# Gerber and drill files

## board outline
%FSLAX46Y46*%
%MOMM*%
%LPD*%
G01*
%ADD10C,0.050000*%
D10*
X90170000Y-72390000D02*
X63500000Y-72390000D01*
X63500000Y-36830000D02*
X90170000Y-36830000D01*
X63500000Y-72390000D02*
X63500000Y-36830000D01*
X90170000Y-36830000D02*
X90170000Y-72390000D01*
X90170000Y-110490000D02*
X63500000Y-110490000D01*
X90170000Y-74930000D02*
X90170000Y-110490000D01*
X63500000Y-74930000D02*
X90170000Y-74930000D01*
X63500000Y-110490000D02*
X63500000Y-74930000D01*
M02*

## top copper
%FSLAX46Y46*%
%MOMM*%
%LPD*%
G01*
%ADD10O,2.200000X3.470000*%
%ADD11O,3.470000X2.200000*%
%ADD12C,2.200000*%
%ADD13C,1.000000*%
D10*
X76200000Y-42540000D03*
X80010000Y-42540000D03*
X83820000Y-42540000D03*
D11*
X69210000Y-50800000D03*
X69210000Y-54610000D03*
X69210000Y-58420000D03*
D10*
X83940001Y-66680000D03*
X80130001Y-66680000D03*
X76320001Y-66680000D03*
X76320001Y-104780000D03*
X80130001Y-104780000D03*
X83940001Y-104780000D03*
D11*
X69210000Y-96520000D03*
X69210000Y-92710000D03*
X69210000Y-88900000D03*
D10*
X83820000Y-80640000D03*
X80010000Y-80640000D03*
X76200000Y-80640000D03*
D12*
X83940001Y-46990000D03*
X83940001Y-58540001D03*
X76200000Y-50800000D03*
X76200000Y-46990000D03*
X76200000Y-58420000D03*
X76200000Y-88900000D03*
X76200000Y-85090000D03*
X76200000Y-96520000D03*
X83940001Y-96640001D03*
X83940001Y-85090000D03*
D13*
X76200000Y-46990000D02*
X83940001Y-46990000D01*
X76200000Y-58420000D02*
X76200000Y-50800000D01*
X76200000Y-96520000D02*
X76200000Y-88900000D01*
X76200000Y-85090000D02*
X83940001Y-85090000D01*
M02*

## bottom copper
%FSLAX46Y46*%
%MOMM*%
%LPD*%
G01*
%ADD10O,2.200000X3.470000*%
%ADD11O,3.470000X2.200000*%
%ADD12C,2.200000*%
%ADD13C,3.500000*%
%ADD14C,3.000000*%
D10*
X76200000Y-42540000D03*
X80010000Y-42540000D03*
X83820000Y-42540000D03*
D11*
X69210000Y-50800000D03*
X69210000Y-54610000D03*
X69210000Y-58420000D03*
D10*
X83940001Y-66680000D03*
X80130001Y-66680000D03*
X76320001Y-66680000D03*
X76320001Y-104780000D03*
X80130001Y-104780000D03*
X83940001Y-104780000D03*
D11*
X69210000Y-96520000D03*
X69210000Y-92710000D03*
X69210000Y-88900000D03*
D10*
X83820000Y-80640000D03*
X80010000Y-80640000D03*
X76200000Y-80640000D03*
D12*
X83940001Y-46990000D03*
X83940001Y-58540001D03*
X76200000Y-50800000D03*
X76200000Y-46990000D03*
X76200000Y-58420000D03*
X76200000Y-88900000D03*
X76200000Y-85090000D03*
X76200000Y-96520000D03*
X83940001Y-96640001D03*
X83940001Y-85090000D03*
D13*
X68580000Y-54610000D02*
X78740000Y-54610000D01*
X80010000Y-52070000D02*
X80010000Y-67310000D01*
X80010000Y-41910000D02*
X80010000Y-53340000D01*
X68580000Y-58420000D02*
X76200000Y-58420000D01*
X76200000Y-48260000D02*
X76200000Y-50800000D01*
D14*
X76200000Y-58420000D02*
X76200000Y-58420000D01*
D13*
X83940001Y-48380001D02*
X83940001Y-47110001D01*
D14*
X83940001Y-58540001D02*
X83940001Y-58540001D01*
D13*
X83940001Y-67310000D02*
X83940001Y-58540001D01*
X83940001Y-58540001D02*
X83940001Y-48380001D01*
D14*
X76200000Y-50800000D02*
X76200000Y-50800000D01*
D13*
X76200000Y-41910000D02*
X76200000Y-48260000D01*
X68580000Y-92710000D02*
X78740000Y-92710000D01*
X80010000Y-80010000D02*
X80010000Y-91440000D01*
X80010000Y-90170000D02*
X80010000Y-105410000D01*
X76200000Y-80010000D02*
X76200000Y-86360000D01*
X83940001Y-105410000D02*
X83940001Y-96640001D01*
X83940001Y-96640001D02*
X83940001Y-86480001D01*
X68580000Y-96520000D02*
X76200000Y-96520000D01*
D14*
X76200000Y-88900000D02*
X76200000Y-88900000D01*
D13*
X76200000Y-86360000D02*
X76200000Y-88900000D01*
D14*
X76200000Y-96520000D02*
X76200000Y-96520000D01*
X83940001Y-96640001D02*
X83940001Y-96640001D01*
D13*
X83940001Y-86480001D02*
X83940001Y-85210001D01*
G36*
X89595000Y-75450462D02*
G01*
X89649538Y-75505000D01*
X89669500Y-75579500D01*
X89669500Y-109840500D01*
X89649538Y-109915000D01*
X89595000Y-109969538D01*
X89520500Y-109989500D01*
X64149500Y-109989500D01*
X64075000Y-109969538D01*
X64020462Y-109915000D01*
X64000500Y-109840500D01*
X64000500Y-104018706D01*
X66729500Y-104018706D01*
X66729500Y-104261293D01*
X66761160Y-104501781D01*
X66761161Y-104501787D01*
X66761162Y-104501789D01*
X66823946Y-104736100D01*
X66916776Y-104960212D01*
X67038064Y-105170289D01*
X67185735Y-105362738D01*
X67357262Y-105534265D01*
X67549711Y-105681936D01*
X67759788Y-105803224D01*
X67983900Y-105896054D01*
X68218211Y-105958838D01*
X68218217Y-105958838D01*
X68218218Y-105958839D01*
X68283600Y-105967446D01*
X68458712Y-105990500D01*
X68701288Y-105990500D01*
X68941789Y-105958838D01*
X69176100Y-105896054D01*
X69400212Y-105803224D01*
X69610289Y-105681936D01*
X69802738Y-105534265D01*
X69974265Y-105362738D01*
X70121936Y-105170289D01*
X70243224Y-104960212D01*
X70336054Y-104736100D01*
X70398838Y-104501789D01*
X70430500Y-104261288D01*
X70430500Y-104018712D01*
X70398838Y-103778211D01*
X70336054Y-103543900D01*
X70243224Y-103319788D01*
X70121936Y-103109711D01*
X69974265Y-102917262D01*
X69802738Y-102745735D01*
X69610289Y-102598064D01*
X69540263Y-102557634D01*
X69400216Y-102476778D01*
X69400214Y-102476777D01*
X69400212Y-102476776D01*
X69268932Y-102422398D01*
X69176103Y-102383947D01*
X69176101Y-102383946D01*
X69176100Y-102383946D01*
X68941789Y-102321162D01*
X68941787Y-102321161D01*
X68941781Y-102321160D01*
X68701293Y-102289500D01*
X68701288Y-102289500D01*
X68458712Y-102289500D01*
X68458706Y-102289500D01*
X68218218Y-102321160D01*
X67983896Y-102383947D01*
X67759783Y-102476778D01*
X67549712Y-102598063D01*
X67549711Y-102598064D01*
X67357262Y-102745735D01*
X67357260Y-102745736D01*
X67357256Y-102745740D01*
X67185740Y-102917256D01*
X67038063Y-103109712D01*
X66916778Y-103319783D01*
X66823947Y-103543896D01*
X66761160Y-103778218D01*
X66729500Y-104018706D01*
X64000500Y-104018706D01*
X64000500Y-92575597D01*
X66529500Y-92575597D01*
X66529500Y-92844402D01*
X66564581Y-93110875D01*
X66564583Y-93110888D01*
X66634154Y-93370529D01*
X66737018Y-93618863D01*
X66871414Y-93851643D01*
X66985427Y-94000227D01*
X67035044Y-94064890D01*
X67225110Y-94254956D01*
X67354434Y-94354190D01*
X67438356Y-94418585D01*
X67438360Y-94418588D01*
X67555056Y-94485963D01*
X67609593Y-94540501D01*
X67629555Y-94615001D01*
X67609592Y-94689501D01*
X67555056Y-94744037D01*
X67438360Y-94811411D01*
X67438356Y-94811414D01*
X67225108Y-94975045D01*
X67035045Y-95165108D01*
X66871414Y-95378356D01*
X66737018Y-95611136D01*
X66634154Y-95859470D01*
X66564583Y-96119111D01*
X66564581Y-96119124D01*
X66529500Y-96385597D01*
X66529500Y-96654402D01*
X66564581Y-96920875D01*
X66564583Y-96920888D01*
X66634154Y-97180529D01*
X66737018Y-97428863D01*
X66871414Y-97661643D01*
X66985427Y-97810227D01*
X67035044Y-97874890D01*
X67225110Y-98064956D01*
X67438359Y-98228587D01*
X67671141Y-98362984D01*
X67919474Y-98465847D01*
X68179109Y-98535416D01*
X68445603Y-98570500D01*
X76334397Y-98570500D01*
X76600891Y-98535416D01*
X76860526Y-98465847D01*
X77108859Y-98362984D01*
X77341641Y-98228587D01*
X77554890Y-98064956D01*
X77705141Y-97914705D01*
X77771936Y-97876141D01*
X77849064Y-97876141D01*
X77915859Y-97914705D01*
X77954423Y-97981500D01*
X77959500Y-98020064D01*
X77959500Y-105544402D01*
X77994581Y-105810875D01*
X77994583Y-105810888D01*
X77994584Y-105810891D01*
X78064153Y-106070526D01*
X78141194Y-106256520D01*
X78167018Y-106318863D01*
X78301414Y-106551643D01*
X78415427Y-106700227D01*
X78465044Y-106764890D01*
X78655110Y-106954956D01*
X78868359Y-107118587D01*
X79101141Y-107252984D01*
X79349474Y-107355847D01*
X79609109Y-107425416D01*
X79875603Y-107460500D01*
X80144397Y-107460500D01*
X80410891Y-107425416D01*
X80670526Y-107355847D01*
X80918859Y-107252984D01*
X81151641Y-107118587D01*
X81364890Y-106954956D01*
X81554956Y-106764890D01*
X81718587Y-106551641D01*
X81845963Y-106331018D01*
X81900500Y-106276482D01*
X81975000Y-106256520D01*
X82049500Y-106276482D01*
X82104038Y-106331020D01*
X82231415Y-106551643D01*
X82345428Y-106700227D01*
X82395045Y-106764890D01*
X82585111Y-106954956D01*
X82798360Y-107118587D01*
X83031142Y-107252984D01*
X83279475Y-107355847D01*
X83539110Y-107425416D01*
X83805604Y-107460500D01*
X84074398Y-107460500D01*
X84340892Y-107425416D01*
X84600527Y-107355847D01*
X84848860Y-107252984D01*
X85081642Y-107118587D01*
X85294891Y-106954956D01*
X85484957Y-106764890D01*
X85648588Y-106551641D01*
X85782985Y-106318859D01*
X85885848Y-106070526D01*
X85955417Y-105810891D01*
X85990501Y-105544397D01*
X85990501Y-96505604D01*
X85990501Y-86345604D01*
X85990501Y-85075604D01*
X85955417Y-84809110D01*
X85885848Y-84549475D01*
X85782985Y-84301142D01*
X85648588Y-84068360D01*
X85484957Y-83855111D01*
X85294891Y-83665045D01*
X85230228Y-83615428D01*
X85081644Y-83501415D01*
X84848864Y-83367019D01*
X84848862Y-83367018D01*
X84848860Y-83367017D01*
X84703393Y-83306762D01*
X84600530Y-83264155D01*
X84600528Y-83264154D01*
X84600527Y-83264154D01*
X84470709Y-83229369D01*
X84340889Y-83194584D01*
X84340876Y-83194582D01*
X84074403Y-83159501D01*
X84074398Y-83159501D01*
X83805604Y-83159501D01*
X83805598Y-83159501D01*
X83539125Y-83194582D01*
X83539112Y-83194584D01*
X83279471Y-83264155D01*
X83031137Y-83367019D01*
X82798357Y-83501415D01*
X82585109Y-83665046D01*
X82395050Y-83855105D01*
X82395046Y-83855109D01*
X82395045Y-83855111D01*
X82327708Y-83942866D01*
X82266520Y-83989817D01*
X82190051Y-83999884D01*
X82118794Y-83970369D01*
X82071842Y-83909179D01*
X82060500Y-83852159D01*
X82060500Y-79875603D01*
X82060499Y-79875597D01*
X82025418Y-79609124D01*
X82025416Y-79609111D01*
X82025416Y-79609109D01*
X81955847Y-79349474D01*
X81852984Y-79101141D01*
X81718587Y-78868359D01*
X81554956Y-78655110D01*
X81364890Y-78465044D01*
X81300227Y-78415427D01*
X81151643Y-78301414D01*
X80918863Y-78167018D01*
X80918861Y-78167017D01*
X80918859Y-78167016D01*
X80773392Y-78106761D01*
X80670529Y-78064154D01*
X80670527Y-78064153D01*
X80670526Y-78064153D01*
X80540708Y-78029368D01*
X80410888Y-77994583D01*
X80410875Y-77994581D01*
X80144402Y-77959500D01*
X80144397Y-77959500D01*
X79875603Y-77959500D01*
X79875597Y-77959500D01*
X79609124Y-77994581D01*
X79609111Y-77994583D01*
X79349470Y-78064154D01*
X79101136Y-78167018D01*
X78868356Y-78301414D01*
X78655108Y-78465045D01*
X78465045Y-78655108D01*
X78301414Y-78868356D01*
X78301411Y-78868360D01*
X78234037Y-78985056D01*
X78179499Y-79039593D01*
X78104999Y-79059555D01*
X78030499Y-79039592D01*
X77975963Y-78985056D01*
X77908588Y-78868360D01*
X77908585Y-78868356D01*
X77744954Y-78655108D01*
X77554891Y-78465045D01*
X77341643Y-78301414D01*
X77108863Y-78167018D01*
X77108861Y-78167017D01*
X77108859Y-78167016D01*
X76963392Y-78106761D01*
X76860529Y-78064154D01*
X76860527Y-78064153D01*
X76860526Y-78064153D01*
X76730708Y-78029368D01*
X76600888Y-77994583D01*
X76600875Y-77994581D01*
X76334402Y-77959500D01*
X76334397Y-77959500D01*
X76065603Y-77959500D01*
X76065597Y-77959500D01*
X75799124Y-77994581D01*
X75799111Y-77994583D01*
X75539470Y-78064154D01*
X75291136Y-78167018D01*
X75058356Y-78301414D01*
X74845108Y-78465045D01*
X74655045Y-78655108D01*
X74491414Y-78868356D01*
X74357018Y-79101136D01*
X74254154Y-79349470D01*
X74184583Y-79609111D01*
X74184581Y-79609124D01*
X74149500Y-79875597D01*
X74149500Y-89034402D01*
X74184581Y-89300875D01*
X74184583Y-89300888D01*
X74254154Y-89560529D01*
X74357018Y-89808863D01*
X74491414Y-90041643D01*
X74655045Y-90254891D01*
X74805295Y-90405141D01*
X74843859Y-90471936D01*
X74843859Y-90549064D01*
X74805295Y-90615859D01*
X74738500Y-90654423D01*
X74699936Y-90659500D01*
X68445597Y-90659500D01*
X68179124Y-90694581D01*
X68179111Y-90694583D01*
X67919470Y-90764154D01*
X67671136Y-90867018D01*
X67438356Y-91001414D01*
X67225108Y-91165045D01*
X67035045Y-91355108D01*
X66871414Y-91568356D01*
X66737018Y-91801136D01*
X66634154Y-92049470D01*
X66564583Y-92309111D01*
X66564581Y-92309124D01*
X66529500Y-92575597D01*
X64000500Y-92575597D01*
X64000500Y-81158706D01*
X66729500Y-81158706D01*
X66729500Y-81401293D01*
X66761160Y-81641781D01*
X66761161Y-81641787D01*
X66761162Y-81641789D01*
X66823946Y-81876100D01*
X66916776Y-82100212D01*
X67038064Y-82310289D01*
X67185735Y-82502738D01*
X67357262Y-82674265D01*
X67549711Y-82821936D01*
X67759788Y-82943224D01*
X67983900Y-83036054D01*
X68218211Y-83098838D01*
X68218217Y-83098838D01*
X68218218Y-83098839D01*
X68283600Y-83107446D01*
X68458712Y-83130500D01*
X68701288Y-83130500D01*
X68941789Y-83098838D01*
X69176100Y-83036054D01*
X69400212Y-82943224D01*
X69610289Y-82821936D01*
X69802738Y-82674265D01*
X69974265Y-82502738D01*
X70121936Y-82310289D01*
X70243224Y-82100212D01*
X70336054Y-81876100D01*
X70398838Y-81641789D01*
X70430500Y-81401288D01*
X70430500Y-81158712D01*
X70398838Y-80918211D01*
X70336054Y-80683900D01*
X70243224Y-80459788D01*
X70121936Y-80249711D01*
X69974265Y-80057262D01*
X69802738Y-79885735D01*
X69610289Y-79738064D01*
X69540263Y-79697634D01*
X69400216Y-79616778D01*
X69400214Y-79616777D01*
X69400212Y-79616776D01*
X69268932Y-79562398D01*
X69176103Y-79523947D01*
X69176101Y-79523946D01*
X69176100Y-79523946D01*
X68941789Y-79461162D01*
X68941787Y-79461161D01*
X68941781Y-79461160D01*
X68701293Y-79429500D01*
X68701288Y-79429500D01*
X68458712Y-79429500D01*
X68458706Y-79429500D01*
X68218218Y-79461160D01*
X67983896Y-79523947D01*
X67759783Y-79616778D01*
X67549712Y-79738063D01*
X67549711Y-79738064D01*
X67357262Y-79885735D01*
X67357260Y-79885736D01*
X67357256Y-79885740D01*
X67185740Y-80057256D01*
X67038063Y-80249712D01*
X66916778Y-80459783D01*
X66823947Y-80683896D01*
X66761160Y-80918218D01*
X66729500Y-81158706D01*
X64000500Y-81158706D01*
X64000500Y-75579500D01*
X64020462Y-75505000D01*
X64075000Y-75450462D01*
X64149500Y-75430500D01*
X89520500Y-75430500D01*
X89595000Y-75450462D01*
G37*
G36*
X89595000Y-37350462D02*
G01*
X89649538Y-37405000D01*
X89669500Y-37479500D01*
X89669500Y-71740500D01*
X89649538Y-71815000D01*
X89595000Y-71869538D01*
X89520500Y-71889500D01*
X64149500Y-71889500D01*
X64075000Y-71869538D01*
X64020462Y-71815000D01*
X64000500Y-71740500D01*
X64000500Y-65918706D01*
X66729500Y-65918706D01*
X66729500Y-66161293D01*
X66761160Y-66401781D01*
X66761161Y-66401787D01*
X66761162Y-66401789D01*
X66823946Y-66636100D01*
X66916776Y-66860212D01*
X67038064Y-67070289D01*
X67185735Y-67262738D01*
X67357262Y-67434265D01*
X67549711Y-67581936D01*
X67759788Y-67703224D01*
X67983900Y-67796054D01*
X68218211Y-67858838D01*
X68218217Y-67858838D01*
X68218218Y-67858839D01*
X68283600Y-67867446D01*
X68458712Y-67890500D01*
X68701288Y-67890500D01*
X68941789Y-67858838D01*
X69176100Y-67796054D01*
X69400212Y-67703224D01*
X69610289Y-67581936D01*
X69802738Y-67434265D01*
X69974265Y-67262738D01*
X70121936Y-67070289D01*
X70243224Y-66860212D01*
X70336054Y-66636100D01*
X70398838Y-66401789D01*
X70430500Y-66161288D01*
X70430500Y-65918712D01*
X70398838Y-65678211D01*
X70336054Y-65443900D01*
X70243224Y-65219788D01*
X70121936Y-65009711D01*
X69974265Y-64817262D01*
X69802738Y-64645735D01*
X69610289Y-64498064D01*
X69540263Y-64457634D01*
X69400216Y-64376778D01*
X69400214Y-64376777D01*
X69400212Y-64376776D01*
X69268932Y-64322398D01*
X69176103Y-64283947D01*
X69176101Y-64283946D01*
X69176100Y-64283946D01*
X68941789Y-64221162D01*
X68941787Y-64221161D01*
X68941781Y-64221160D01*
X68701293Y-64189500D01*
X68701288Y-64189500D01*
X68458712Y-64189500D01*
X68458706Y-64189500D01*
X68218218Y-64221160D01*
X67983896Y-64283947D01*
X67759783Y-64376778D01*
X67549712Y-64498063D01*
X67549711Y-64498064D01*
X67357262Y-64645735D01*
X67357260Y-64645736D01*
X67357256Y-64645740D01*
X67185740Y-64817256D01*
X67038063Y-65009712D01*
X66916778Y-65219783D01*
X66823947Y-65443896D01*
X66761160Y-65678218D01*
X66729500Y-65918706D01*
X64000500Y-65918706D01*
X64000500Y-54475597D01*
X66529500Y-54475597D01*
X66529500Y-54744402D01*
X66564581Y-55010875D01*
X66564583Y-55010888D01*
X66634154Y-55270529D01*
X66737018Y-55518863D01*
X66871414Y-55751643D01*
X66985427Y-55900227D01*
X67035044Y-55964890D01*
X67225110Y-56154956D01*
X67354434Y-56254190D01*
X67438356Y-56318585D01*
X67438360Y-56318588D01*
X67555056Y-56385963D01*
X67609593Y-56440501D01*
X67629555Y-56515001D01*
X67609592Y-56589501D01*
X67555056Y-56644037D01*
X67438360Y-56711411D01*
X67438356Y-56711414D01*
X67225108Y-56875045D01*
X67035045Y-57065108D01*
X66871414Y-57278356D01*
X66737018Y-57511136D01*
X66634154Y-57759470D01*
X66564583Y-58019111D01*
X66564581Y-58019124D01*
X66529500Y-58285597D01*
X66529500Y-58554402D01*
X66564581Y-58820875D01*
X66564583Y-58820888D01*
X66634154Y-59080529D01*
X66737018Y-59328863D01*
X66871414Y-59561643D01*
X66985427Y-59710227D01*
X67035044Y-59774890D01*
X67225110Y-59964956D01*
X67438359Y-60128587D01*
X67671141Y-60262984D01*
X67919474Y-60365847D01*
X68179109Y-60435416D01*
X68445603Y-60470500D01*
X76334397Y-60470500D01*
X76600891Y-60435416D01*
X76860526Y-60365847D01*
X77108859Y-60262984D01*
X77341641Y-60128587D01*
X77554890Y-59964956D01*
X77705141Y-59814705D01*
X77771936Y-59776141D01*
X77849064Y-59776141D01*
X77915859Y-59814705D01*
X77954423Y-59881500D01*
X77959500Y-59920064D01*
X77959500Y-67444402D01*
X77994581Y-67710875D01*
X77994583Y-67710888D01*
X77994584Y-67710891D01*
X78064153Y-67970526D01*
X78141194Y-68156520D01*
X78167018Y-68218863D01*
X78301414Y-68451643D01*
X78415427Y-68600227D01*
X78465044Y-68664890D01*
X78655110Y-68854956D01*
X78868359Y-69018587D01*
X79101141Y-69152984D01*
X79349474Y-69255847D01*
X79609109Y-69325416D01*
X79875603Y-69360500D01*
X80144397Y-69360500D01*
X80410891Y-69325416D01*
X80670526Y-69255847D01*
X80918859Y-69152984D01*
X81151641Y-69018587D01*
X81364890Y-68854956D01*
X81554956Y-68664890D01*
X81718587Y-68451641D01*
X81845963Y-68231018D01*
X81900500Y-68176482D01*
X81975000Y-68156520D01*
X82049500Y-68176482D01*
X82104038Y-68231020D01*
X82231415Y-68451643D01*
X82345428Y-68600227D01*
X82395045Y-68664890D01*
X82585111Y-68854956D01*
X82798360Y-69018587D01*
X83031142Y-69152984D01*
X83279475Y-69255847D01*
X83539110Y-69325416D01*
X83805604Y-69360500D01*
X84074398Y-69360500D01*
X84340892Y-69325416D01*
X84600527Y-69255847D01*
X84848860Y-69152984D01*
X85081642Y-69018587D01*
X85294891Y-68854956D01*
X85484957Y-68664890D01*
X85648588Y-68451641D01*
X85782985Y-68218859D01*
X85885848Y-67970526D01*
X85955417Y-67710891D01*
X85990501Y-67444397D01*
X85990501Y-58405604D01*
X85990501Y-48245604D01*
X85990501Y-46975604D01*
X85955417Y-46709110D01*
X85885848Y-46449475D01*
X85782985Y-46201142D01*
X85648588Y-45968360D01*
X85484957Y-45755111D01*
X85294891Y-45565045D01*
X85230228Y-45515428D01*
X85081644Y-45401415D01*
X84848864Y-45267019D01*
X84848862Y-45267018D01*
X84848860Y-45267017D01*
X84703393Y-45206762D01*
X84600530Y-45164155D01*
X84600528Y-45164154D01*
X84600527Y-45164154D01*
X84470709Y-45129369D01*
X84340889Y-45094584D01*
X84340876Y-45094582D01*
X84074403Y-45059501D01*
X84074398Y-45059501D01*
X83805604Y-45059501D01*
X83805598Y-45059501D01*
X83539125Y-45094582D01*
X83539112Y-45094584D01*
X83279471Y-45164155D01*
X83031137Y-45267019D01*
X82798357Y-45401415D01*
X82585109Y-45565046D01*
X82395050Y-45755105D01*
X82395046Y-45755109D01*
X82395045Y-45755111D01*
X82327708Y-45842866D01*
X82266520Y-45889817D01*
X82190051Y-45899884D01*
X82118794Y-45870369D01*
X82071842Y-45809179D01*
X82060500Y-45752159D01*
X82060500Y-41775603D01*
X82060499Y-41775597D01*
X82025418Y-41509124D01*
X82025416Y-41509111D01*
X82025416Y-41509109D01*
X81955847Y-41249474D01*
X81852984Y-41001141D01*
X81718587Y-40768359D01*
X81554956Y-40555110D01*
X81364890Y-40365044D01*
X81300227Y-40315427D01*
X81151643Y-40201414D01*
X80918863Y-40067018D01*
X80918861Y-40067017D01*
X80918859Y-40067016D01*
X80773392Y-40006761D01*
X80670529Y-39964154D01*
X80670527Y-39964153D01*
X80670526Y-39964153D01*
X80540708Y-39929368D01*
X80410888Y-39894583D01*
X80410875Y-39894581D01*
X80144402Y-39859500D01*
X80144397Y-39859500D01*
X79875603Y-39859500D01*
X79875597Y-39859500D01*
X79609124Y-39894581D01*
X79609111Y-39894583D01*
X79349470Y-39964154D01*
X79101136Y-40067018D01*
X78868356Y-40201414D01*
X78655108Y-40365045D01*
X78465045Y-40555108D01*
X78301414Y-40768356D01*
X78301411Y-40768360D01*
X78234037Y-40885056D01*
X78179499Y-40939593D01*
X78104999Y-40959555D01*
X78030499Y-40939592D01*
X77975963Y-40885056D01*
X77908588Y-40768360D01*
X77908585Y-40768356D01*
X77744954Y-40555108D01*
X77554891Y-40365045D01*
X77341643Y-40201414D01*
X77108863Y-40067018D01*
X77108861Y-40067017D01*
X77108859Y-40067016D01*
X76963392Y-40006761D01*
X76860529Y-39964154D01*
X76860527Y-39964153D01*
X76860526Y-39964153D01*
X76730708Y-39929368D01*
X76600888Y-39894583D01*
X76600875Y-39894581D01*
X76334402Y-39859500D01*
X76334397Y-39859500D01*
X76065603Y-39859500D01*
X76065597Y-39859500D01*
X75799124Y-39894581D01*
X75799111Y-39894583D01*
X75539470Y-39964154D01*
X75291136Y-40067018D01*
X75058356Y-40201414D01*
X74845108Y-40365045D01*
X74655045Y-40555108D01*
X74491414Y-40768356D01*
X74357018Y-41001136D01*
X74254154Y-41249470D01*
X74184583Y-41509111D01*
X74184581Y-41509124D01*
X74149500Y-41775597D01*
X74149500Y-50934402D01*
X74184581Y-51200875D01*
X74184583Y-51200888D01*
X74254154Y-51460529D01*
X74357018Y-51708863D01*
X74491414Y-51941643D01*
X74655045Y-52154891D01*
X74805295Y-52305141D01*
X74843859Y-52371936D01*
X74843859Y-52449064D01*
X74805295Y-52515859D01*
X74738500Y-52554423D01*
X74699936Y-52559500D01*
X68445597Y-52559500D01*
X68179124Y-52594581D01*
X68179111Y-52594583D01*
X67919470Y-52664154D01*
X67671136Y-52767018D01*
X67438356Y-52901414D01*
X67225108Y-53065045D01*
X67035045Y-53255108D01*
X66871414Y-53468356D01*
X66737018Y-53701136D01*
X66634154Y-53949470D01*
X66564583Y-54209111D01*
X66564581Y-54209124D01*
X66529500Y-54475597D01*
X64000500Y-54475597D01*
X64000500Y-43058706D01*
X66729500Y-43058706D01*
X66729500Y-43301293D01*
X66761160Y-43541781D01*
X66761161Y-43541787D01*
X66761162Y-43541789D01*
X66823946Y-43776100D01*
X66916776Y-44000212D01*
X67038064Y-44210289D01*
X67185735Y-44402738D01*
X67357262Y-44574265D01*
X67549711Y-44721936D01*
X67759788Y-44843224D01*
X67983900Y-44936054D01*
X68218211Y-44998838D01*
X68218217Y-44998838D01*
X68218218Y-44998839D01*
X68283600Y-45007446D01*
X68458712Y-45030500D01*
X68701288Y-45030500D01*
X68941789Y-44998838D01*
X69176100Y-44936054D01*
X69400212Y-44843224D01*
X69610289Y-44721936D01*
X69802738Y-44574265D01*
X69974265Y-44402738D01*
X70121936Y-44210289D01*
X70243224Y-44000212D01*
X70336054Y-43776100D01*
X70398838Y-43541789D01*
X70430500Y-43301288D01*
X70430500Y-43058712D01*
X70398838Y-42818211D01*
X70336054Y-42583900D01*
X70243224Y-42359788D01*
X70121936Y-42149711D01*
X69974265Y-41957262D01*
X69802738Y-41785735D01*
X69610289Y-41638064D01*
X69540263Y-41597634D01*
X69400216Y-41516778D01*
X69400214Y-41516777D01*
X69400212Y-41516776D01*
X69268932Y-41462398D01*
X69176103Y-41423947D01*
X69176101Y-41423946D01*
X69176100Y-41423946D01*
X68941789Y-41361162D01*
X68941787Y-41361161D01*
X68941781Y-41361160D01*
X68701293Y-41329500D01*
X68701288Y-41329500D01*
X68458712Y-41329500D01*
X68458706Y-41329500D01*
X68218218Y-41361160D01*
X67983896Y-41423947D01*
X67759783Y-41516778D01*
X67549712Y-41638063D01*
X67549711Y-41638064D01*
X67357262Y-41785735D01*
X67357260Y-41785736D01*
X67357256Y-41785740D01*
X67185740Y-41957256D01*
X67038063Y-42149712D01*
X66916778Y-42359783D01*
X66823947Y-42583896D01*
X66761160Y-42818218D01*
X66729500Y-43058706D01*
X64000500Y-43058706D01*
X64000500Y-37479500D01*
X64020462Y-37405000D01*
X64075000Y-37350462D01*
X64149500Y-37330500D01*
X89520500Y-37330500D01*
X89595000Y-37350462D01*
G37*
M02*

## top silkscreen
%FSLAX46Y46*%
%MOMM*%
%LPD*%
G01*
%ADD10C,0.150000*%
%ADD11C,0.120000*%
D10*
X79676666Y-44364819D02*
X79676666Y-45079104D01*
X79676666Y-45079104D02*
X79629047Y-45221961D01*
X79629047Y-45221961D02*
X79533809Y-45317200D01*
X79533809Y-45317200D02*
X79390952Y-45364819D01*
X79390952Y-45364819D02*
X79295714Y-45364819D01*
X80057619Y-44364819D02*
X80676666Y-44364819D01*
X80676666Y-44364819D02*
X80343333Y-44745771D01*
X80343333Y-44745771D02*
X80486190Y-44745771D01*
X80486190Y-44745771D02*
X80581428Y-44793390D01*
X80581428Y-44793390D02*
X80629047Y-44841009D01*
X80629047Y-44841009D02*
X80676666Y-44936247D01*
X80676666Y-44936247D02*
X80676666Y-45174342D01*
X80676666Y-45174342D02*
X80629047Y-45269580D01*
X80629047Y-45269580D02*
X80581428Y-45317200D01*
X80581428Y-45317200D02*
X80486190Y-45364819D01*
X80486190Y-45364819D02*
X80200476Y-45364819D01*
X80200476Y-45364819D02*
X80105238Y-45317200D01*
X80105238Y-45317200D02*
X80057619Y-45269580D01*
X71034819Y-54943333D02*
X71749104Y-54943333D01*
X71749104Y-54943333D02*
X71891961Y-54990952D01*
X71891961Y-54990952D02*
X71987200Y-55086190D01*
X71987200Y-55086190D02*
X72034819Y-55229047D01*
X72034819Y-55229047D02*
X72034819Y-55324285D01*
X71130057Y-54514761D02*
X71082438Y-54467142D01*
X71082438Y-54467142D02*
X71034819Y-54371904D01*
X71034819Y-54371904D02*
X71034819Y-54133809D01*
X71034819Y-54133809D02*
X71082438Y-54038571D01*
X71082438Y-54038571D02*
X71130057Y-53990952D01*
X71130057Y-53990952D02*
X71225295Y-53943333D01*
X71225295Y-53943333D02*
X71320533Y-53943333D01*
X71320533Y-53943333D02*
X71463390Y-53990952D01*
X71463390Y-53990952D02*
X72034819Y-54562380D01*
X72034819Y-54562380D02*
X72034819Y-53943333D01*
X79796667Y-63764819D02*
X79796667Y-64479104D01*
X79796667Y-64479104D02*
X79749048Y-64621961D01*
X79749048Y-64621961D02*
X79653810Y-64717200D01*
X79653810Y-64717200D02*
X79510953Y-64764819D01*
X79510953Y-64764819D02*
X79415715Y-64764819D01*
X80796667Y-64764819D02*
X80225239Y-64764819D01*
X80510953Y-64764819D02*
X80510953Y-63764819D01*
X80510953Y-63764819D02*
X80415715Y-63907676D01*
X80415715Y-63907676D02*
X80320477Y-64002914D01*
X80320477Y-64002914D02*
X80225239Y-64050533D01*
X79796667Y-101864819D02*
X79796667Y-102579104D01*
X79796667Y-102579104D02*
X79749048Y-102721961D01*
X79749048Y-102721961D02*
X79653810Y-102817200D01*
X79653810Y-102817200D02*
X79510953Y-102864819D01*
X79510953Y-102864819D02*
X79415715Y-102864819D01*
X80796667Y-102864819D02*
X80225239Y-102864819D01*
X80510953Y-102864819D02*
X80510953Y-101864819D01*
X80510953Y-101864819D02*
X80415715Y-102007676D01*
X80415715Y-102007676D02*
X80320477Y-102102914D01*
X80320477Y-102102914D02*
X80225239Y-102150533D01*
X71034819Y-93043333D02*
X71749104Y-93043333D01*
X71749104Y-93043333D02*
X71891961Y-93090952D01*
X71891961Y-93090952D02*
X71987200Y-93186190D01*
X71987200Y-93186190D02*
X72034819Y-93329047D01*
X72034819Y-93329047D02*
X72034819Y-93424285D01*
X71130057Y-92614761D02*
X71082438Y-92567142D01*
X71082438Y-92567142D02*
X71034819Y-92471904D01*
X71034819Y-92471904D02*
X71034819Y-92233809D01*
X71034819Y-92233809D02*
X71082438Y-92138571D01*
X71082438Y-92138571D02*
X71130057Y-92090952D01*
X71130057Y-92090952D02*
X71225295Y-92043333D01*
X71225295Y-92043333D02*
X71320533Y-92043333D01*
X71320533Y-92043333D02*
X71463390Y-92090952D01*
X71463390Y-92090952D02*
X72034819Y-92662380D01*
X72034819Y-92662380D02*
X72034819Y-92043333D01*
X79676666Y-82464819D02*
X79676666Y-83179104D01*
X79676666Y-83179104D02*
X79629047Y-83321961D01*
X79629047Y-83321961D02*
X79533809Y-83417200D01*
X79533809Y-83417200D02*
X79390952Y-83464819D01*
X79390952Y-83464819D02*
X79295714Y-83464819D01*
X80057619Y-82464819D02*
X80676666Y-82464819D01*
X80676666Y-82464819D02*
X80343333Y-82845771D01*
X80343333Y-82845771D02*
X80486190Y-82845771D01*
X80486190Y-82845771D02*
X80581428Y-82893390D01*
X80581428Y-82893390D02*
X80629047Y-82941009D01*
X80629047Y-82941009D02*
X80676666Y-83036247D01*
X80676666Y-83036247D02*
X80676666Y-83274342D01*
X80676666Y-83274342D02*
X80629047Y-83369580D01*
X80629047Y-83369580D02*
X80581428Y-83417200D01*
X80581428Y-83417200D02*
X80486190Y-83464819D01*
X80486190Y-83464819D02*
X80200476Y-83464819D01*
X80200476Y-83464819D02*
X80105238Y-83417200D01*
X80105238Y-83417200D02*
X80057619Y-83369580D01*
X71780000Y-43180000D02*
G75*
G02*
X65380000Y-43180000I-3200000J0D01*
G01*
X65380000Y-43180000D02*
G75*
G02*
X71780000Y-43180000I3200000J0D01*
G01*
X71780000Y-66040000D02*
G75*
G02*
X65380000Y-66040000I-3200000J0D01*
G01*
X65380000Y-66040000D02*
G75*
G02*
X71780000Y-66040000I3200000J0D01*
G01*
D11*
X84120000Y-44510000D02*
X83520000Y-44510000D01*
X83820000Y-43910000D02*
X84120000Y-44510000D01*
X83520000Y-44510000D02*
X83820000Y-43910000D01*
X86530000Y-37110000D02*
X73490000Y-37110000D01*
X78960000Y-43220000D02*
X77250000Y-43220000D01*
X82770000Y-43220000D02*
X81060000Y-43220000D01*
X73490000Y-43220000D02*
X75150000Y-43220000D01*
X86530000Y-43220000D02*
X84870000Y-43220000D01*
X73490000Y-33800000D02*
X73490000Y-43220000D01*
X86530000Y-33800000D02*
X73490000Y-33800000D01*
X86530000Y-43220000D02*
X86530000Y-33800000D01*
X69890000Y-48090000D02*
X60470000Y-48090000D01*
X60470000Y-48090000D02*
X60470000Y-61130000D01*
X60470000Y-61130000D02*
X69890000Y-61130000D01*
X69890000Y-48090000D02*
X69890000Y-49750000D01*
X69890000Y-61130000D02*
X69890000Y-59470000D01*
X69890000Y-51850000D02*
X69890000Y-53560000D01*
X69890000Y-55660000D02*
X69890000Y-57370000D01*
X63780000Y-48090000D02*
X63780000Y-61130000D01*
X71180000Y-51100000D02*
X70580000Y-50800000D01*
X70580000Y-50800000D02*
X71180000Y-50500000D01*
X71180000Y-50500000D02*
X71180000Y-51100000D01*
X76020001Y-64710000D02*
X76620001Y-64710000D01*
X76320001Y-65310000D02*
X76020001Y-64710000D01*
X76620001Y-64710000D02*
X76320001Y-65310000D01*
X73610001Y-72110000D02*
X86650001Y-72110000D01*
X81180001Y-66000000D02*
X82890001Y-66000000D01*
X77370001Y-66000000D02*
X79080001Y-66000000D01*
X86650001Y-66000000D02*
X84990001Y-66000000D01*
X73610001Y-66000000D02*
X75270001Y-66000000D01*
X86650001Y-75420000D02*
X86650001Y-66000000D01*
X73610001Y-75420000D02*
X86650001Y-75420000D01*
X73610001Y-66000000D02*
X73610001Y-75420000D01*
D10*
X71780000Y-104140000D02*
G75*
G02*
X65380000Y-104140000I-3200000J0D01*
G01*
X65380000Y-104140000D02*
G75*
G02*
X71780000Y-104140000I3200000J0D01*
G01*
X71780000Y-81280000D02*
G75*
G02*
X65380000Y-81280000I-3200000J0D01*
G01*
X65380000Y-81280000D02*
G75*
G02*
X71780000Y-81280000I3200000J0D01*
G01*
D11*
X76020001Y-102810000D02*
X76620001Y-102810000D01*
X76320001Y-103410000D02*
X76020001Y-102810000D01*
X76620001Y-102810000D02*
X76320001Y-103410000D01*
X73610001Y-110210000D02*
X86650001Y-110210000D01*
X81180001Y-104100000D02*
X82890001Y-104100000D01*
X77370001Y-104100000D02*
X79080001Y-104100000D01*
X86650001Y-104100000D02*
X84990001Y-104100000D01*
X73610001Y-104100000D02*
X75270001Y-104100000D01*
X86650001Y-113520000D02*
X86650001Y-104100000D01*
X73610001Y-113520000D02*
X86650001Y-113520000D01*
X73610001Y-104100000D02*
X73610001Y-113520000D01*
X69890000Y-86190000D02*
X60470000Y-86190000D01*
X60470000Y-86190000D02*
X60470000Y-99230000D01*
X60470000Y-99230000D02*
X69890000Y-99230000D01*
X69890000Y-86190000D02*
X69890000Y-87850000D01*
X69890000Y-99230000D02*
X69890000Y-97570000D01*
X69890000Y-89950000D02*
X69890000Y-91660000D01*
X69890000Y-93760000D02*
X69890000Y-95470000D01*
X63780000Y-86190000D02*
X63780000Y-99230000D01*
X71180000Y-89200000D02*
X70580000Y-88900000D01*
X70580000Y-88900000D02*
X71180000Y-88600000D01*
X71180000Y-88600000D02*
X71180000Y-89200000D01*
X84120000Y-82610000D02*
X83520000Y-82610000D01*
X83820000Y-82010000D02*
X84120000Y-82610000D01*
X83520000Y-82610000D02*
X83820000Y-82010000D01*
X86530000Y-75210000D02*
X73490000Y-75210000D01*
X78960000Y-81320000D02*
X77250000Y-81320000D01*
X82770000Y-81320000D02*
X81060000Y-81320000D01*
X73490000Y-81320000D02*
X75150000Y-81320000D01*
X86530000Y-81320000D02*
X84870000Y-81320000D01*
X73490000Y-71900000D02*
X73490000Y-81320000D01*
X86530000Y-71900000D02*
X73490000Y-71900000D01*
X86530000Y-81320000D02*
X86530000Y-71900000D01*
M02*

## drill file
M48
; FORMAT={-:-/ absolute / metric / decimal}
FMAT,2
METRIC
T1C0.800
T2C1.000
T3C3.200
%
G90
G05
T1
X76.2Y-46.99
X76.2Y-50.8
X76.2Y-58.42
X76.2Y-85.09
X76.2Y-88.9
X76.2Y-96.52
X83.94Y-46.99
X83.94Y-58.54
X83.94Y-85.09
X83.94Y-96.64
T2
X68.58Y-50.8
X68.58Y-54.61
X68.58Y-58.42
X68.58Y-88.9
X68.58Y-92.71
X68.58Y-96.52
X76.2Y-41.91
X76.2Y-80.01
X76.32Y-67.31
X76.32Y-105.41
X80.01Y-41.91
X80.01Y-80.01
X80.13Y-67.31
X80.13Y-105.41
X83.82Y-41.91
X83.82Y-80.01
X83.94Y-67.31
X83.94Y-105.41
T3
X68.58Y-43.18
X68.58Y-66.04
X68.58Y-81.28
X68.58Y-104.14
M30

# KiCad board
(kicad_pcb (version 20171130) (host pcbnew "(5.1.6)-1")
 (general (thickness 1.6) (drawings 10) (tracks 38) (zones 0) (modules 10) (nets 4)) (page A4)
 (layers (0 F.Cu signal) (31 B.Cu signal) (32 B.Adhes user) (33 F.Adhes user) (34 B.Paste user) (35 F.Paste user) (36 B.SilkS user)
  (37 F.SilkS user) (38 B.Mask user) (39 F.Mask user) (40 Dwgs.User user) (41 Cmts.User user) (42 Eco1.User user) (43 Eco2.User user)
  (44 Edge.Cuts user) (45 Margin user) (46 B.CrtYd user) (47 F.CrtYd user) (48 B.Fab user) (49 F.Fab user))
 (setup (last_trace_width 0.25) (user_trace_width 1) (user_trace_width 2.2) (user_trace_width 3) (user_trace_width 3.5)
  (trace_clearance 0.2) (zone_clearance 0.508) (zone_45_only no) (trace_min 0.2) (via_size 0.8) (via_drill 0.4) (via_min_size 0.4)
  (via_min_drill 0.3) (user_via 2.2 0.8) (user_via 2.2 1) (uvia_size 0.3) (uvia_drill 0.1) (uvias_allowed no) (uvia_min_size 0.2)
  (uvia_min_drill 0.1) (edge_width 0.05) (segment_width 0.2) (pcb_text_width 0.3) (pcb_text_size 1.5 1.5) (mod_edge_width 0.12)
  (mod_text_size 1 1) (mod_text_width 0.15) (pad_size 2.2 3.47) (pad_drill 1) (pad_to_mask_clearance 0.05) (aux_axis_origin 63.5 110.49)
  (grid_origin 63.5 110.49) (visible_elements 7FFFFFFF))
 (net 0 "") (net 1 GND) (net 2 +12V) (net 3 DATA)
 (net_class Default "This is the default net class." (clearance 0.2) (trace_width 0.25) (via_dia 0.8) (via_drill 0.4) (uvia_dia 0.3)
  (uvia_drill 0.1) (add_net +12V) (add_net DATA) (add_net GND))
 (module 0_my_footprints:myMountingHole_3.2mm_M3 (layer F.Cu) (at 68.58 43.18 90)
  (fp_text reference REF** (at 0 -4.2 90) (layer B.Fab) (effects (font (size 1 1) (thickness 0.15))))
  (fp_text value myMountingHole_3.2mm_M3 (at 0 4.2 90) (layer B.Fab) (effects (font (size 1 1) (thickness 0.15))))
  (fp_circle (center 0 0) (end 3.2 0) (layer F.SilkS) (width 0.15))
  (pad "" np_thru_hole circle (at 0 0 90) (size 3.2 3.2) (drill 3.2) (layers *.Cu *.Mask)))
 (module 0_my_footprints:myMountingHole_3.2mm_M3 (layer F.Cu) (at 68.58 66.04 90)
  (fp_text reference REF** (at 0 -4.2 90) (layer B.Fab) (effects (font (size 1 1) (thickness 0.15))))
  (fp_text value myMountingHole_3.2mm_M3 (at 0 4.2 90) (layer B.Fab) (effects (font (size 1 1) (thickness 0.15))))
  (fp_circle (center 0 0) (end 3.2 0) (layer F.SilkS) (width 0.15))
  (pad "" np_thru_hole circle (at 0 0 90) (size 3.2 3.2) (drill 3.2) (layers *.Cu *.Mask)))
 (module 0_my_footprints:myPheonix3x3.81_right (layer F.Cu) (at 83.82 41.91 180)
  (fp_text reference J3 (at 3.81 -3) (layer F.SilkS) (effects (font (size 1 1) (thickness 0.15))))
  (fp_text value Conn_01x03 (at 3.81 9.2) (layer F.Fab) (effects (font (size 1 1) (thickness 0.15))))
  (fp_line (start -0.3 -2.6) (end 0.3 -2.6) (layer F.SilkS) (width 0.12))
  (fp_line (start 0 -2) (end -0.3 -2.6) (layer F.SilkS) (width 0.12))
  (fp_line (start 0.3 -2.6) (end 0 -2) (layer F.SilkS) (width 0.12))
  (fp_line (start -2.71 4.8) (end 10.33 4.8) (layer F.SilkS) (width 0.12))
  (fp_line (start 4.86 -1.31) (end 6.57 -1.31) (layer F.SilkS) (width 0.12))
  (fp_line (start 1.05 -1.31) (end 2.76 -1.31) (layer F.SilkS) (width 0.12))
  (fp_line (start 10.33 -1.31) (end 8.67 -1.31) (layer F.SilkS) (width 0.12))
  (fp_line (start -2.71 -1.31) (end -1.05 -1.31) (layer F.SilkS) (width 0.12))
  (fp_line (start 10.33 8.11) (end 10.33 -1.31) (layer F.SilkS) (width 0.12))
  (fp_line (start -2.71 8.11) (end 10.33 8.11) (layer F.SilkS) (width 0.12))
  (fp_line (start -2.71 -1.31) (end -2.71 8.11) (layer F.SilkS) (width 0.12))
  (pad 3 thru_hole oval (at 7.62 0 180) (size 2.2 3.47) (drill 1 (offset 0 -0.63)) (layers *.Cu *.Mask))
  (pad 2 thru_hole oval (at 3.81 0 180) (size 2.2 3.47) (drill 1 (offset 0 -0.63)) (layers *.Cu *.Mask))
  (pad 1 thru_hole oval (at 0 0 180) (size 2.2 3.47) (drill 1 (offset 0 -0.63)) (layers *.Cu *.Mask) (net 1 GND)))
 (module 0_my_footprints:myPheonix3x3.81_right (layer F.Cu) (at 68.58 50.8 270)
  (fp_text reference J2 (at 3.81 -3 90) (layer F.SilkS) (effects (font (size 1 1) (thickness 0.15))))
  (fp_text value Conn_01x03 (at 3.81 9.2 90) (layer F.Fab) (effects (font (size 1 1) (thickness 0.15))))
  (fp_line (start -2.71 -1.31) (end -2.71 8.11) (layer F.SilkS) (width 0.12))
  (fp_line (start -2.71 8.11) (end 10.33 8.11) (layer F.SilkS) (width 0.12))
  (fp_line (start 10.33 8.11) (end 10.33 -1.31) (layer F.SilkS) (width 0.12))
  (fp_line (start -2.71 -1.31) (end -1.05 -1.31) (layer F.SilkS) (width 0.12))
  (fp_line (start 10.33 -1.31) (end 8.67 -1.31) (layer F.SilkS) (width 0.12))
  (fp_line (start 1.05 -1.31) (end 2.76 -1.31) (layer F.SilkS) (width 0.12))
  (fp_line (start 4.86 -1.31) (end 6.57 -1.31) (layer F.SilkS) (width 0.12))
  (fp_line (start -2.71 4.8) (end 10.33 4.8) (layer F.SilkS) (width 0.12))
  (fp_line (start 0.3 -2.6) (end 0 -2) (layer F.SilkS) (width 0.12))
  (fp_line (start 0 -2) (end -0.3 -2.6) (layer F.SilkS) (width 0.12))
  (fp_line (start -0.3 -2.6) (end 0.3 -2.6) (layer F.SilkS) (width 0.12))
  (pad 1 thru_hole oval (at 0 0 270) (size 2.2 3.47) (drill 1 (offset 0 -0.63)) (layers *.Cu *.Mask) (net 1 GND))
  (pad 2 thru_hole oval (at 3.81 0 270) (size 2.2 3.47) (drill 1 (offset 0 -0.63)) (layers *.Cu *.Mask))
  (pad 3 thru_hole oval (at 7.62 0 270) (size 2.2 3.47) (drill 1 (offset 0 -0.63)) (layers *.Cu *.Mask)))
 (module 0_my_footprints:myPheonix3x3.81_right (layer F.Cu) (at 76.320001 67.31)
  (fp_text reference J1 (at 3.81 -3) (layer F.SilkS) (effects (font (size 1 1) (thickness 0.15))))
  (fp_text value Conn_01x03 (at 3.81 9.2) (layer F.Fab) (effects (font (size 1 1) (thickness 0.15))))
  (fp_line (start -0.3 -2.6) (end 0.3 -2.6) (layer F.SilkS) (width 0.12))
  (fp_line (start 0 -2) (end -0.3 -2.6) (layer F.SilkS) (width 0.12))
  (fp_line (start 0.3 -2.6) (end 0 -2) (layer F.SilkS) (width 0.12))
  (fp_line (start -2.71 4.8) (end 10.33 4.8) (layer F.SilkS) (width 0.12))
  (fp_line (start 4.86 -1.31) (end 6.57 -1.31) (layer F.SilkS) (width 0.12))
  (fp_line (start 1.05 -1.31) (end 2.76 -1.31) (layer F.SilkS) (width 0.12))
  (fp_line (start 10.33 -1.31) (end 8.67 -1.31) (layer F.SilkS) (width 0.12))
  (fp_line (start -2.71 -1.31) (end -1.05 -1.31) (layer F.SilkS) (width 0.12))
  (fp_line (start 10.33 8.11) (end 10.33 -1.31) (layer F.SilkS) (width 0.12))
  (fp_line (start -2.71 8.11) (end 10.33 8.11) (layer F.SilkS) (width 0.12))
  (fp_line (start -2.71 -1.31) (end -2.71 8.11) (layer F.SilkS) (width 0.12))
  (pad 3 thru_hole oval (at 7.62 0) (size 2.2 3.47) (drill 1 (offset 0 -0.63)) (layers *.Cu *.Mask))
  (pad 2 thru_hole oval (at 3.81 0) (size 2.2 3.47) (drill 1 (offset 0 -0.63)) (layers *.Cu *.Mask))
  (pad 1 thru_hole oval (at 0 0) (size 2.2 3.47) (drill 1 (offset 0 -0.63)) (layers *.Cu *.Mask) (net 1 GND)))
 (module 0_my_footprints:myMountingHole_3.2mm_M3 (layer F.Cu) (at 68.58 104.14 90)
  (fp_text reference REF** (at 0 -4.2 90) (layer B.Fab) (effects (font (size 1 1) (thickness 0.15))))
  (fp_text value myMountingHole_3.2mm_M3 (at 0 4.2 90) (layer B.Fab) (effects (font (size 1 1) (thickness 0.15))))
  (fp_circle (center 0 0) (end 3.2 0) (layer F.SilkS) (width 0.15))
  (pad "" np_thru_hole circle (at 0 0 90) (size 3.2 3.2) (drill 3.2) (layers *.Cu *.Mask)))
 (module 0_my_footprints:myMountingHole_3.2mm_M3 (layer F.Cu) (at 68.58 81.28 90)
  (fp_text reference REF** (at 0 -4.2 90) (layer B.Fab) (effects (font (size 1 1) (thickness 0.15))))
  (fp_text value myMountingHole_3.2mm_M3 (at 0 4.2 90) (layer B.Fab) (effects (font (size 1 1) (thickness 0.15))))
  (fp_circle (center 0 0) (end 3.2 0) (layer F.SilkS) (width 0.15))
  (pad "" np_thru_hole circle (at 0 0 90) (size 3.2 3.2) (drill 3.2) (layers *.Cu *.Mask)))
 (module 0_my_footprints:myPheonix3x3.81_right (layer F.Cu) (at 76.320001 105.41)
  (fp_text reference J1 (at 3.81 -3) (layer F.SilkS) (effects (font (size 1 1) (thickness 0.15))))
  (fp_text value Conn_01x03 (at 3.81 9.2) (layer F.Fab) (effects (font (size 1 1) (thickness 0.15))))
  (fp_line (start -0.3 -2.6) (end 0.3 -2.6) (layer F.SilkS) (width 0.12))
  (fp_line (start 0 -2) (end -0.3 -2.6) (layer F.SilkS) (width 0.12))
  (fp_line (start 0.3 -2.6) (end 0 -2) (layer F.SilkS) (width 0.12))
  (fp_line (start -2.71 4.8) (end 10.33 4.8) (layer F.SilkS) (width 0.12))
  (fp_line (start 4.86 -1.31) (end 6.57 -1.31) (layer F.SilkS) (width 0.12))
  (fp_line (start 1.05 -1.31) (end 2.76 -1.31) (layer F.SilkS) (width 0.12))
  (fp_line (start 10.33 -1.31) (end 8.67 -1.31) (layer F.SilkS) (width 0.12))
  (fp_line (start -2.71 -1.31) (end -1.05 -1.31) (layer F.SilkS) (width 0.12))
  (fp_line (start 10.33 8.11) (end 10.33 -1.31) (layer F.SilkS) (width 0.12))
  (fp_line (start -2.71 8.11) (end 10.33 8.11) (layer F.SilkS) (width 0.12))
  (fp_line (start -2.71 -1.31) (end -2.71 8.11) (layer F.SilkS) (width 0.12))
  (pad 1 thru_hole oval (at 0 0) (size 2.2 3.47) (drill 1 (offset 0 -0.63)) (layers *.Cu *.Mask) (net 1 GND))
  (pad 2 thru_hole oval (at 3.81 0) (size 2.2 3.47) (drill 1 (offset 0 -0.63)) (layers *.Cu *.Mask) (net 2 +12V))
  (pad 3 thru_hole oval (at 7.62 0) (size 2.2 3.47) (drill 1 (offset 0 -0.63)) (layers *.Cu *.Mask) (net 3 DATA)))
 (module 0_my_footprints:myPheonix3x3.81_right (layer F.Cu) (at 68.58 88.9 270)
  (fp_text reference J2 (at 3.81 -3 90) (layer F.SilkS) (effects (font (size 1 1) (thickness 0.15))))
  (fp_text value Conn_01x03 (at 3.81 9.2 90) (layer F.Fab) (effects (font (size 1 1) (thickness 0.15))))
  (fp_line (start -2.71 -1.31) (end -2.71 8.11) (layer F.SilkS) (width 0.12))
  (fp_line (start -2.71 8.11) (end 10.33 8.11) (layer F.SilkS) (width 0.12))
  (fp_line (start 10.33 8.11) (end 10.33 -1.31) (layer F.SilkS) (width 0.12))
  (fp_line (start -2.71 -1.31) (end -1.05 -1.31) (layer F.SilkS) (width 0.12))
  (fp_line (start 10.33 -1.31) (end 8.67 -1.31) (layer F.SilkS) (width 0.12))
  (fp_line (start 1.05 -1.31) (end 2.76 -1.31) (layer F.SilkS) (width 0.12))
  (fp_line (start 4.86 -1.31) (end 6.57 -1.31) (layer F.SilkS) (width 0.12))
  (fp_line (start -2.71 4.8) (end 10.33 4.8) (layer F.SilkS) (width 0.12))
  (fp_line (start 0.3 -2.6) (end 0 -2) (layer F.SilkS) (width 0.12))
  (fp_line (start 0 -2) (end -0.3 -2.6) (layer F.SilkS) (width 0.12))
  (fp_line (start -0.3 -2.6) (end 0.3 -2.6) (layer F.SilkS) (width 0.12))
  (pad 3 thru_hole oval (at 7.62 0 270) (size 2.2 3.47) (drill 1 (offset 0 -0.63)) (layers *.Cu *.Mask) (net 3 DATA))
  (pad 2 thru_hole oval (at 3.81 0 270) (size 2.2 3.47) (drill 1 (offset 0 -0.63)) (layers *.Cu *.Mask) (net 2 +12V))
  (pad 1 thru_hole oval (at 0 0 270) (size 2.2 3.47) (drill 1 (offset 0 -0.63)) (layers *.Cu *.Mask) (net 1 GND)))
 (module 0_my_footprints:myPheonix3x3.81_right (layer F.Cu) (at 83.82 80.01 180)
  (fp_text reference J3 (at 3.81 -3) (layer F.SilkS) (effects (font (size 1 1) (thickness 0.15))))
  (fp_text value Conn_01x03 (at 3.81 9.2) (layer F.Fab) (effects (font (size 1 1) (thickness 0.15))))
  (fp_line (start -0.3 -2.6) (end 0.3 -2.6) (layer F.SilkS) (width 0.12))
  (fp_line (start 0 -2) (end -0.3 -2.6) (layer F.SilkS) (width 0.12))
  (fp_line (start 0.3 -2.6) (end 0 -2) (layer F.SilkS) (width 0.12))
  (fp_line (start -2.71 4.8) (end 10.33 4.8) (layer F.SilkS) (width 0.12))
  (fp_line (start 4.86 -1.31) (end 6.57 -1.31) (layer F.SilkS) (width 0.12))
  (fp_line (start 1.05 -1.31) (end 2.76 -1.31) (layer F.SilkS) (width 0.12))
  (fp_line (start 10.33 -1.31) (end 8.67 -1.31) (layer F.SilkS) (width 0.12))
  (fp_line (start -2.71 -1.31) (end -1.05 -1.31) (layer F.SilkS) (width 0.12))
  (fp_line (start 10.33 8.11) (end 10.33 -1.31) (layer F.SilkS) (width 0.12))
  (fp_line (start -2.71 8.11) (end 10.33 8.11) (layer F.SilkS) (width 0.12))
  (fp_line (start -2.71 -1.31) (end -2.71 8.11) (layer F.SilkS) (width 0.12))
  (pad 1 thru_hole oval (at 0 0 180) (size 2.2 3.47) (drill 1 (offset 0 -0.63)) (layers *.Cu *.Mask) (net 1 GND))
  (pad 2 thru_hole oval (at 3.81 0 180) (size 2.2 3.47) (drill 1 (offset 0 -0.63)) (layers *.Cu *.Mask) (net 2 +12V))
  (pad 3 thru_hole oval (at 7.62 0 180) (size 2.2 3.47) (drill 1 (offset 0 -0.63)) (layers *.Cu *.Mask) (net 3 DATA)))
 (gr_line (start 90.17 72.39) (end 63.5 72.39) (layer Edge.Cuts) (width 0.05))
 (gr_line (start 63.5 36.83) (end 90.17 36.83) (layer Edge.Cuts) (width 0.05))
 (gr_line (start 63.5 72.39) (end 63.5 36.83) (layer Edge.Cuts) (width 0.05))
 (gr_line (start 90.17 36.83) (end 90.17 72.39) (layer Edge.Cuts) (width 0.05))
 (gr_line (start 90.17 110.49) (end 63.5 110.49) (layer Edge.Cuts) (width 0.05))
 (gr_line (start 90.17 74.93) (end 90.17 110.49) (layer Edge.Cuts) (width 0.05))
 (gr_line (start 63.5 74.93) (end 90.17 74.93) (layer Edge.Cuts) (width 0.05))
 (gr_line (start 63.5 110.49) (end 63.5 74.93) (layer Edge.Cuts) (width 0.05))
 (segment (start 68.58 54.61) (end 78.74 54.61) (width 3.5) (layer B.Cu) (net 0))
 (segment (start 80.01 52.07) (end 80.01 67.31) (width 3.5) (layer B.Cu) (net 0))
 (segment (start 80.01 41.91) (end 80.01 53.34) (width 3.5) (layer B.Cu) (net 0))
 (segment (start 76.2 46.99) (end 83.940001 46.99) (width 1) (layer F.Cu) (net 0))
 (segment (start 76.2 58.42) (end 76.2 50.8) (width 1) (layer F.Cu) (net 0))
 (segment (start 68.58 58.42) (end 76.2 58.42) (width 3.5) (layer B.Cu) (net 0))
 (segment (start 76.2 48.26) (end 76.2 50.8) (width 3.5) (layer B.Cu) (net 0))
 (segment (start 76.2 58.42) (end 76.2 58.42) (width 3) (layer B.Cu) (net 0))
 (segment (start 83.940001 48.380001) (end 83.940001 47.110001) (width 3.5) (layer B.Cu) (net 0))
 (segment (start 83.940001 58.540001) (end 83.940001 58.540001) (width 3) (layer B.Cu) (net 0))
 (segment (start 83.940001 67.31) (end 83.940001 58.540001) (width 3.5) (layer B.Cu) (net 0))
 (segment (start 83.940001 58.540001) (end 83.940001 48.380001) (width 3.5) (layer B.Cu) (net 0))
 (segment (start 76.2 50.8) (end 76.2 50.8) (width 3) (layer B.Cu) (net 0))
 (segment (start 76.2 41.91) (end 76.2 48.26) (width 3.5) (layer B.Cu) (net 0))
 (via (at 83.940001 46.99) (size 2.2) (drill 0.8) (layers F.Cu B.Cu) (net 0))
 (via (at 83.940001 58.540001) (size 2.2) (drill 0.8) (layers F.Cu B.Cu) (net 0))
 (via (at 76.2 50.8) (size 2.2) (drill 0.8) (layers F.Cu B.Cu) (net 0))
 (via (at 76.2 46.99) (size 2.2) (drill 0.8) (layers F.Cu B.Cu) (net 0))
 (via (at 76.2 58.42) (size 2.2) (drill 0.8) (layers F.Cu B.Cu) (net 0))
 (segment (start 68.58 92.71) (end 78.74 92.71) (width 3.5) (layer B.Cu) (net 2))
 (segment (start 80.01 80.01) (end 80.01 91.44) (width 3.5) (layer B.Cu) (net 2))
 (segment (start 80.01 90.17) (end 80.01 105.41) (width 3.5) (layer B.Cu) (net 2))
 (segment (start 76.2 80.01) (end 76.2 86.36) (width 3.5) (layer B.Cu) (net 3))
 (segment (start 83.940001 105.41) (end 83.940001 96.640001) (width 3.5) (layer B.Cu) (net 3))
 (segment (start 83.940001 96.640001) (end 83.940001 86.480001) (width 3.5) (layer B.Cu) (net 3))
 (segment (start 68.58 96.52) (end 76.2 96.52) (width 3.5) (layer B.Cu) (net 3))
 (segment (start 76.2 88.9) (end 76.2 88.9) (width 3) (layer B.Cu) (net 3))
 (via (at 76.2 88.9) (size 2.2) (drill 0.8) (layers F.Cu B.Cu) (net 3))
 (segment (start 76.2 86.36) (end 76.2 88.9) (width 3.5) (layer B.Cu) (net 3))
 (via (at 76.2 85.09) (size 2.2) (drill 0.8) (layers F.Cu B.Cu) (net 3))
 (segment (start 76.2 96.52) (end 76.2 96.52) (width 3) (layer B.Cu) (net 3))
 (via (at 76.2 96.52) (size 2.2) (drill 0.8) (layers F.Cu B.Cu) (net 3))
 (segment (start 83.940001 96.640001) (end 83.940001 96.640001) (width 3) (layer B.Cu) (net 3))
 (via (at 83.940001 96.640001) (size 2.2) (drill 0.8) (layers F.Cu B.Cu) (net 3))
 (segment (start 83.940001 86.480001) (end 83.940001 85.210001) (width 3.5) (layer B.Cu) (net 3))
 (via (at 83.940001 85.09) (size 2.2) (drill 0.8) (layers F.Cu B.Cu) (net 3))
 (segment (start 76.2 96.52) (end 76.2 88.9) (width 1) (layer F.Cu) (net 3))
 (segment (start 76.2 85.09) (end 83.940001 85.09) (width 1) (layer F.Cu) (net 3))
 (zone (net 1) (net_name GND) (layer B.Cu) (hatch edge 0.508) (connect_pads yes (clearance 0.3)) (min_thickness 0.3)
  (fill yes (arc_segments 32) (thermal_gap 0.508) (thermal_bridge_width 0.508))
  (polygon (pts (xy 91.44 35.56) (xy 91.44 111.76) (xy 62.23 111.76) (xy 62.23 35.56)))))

